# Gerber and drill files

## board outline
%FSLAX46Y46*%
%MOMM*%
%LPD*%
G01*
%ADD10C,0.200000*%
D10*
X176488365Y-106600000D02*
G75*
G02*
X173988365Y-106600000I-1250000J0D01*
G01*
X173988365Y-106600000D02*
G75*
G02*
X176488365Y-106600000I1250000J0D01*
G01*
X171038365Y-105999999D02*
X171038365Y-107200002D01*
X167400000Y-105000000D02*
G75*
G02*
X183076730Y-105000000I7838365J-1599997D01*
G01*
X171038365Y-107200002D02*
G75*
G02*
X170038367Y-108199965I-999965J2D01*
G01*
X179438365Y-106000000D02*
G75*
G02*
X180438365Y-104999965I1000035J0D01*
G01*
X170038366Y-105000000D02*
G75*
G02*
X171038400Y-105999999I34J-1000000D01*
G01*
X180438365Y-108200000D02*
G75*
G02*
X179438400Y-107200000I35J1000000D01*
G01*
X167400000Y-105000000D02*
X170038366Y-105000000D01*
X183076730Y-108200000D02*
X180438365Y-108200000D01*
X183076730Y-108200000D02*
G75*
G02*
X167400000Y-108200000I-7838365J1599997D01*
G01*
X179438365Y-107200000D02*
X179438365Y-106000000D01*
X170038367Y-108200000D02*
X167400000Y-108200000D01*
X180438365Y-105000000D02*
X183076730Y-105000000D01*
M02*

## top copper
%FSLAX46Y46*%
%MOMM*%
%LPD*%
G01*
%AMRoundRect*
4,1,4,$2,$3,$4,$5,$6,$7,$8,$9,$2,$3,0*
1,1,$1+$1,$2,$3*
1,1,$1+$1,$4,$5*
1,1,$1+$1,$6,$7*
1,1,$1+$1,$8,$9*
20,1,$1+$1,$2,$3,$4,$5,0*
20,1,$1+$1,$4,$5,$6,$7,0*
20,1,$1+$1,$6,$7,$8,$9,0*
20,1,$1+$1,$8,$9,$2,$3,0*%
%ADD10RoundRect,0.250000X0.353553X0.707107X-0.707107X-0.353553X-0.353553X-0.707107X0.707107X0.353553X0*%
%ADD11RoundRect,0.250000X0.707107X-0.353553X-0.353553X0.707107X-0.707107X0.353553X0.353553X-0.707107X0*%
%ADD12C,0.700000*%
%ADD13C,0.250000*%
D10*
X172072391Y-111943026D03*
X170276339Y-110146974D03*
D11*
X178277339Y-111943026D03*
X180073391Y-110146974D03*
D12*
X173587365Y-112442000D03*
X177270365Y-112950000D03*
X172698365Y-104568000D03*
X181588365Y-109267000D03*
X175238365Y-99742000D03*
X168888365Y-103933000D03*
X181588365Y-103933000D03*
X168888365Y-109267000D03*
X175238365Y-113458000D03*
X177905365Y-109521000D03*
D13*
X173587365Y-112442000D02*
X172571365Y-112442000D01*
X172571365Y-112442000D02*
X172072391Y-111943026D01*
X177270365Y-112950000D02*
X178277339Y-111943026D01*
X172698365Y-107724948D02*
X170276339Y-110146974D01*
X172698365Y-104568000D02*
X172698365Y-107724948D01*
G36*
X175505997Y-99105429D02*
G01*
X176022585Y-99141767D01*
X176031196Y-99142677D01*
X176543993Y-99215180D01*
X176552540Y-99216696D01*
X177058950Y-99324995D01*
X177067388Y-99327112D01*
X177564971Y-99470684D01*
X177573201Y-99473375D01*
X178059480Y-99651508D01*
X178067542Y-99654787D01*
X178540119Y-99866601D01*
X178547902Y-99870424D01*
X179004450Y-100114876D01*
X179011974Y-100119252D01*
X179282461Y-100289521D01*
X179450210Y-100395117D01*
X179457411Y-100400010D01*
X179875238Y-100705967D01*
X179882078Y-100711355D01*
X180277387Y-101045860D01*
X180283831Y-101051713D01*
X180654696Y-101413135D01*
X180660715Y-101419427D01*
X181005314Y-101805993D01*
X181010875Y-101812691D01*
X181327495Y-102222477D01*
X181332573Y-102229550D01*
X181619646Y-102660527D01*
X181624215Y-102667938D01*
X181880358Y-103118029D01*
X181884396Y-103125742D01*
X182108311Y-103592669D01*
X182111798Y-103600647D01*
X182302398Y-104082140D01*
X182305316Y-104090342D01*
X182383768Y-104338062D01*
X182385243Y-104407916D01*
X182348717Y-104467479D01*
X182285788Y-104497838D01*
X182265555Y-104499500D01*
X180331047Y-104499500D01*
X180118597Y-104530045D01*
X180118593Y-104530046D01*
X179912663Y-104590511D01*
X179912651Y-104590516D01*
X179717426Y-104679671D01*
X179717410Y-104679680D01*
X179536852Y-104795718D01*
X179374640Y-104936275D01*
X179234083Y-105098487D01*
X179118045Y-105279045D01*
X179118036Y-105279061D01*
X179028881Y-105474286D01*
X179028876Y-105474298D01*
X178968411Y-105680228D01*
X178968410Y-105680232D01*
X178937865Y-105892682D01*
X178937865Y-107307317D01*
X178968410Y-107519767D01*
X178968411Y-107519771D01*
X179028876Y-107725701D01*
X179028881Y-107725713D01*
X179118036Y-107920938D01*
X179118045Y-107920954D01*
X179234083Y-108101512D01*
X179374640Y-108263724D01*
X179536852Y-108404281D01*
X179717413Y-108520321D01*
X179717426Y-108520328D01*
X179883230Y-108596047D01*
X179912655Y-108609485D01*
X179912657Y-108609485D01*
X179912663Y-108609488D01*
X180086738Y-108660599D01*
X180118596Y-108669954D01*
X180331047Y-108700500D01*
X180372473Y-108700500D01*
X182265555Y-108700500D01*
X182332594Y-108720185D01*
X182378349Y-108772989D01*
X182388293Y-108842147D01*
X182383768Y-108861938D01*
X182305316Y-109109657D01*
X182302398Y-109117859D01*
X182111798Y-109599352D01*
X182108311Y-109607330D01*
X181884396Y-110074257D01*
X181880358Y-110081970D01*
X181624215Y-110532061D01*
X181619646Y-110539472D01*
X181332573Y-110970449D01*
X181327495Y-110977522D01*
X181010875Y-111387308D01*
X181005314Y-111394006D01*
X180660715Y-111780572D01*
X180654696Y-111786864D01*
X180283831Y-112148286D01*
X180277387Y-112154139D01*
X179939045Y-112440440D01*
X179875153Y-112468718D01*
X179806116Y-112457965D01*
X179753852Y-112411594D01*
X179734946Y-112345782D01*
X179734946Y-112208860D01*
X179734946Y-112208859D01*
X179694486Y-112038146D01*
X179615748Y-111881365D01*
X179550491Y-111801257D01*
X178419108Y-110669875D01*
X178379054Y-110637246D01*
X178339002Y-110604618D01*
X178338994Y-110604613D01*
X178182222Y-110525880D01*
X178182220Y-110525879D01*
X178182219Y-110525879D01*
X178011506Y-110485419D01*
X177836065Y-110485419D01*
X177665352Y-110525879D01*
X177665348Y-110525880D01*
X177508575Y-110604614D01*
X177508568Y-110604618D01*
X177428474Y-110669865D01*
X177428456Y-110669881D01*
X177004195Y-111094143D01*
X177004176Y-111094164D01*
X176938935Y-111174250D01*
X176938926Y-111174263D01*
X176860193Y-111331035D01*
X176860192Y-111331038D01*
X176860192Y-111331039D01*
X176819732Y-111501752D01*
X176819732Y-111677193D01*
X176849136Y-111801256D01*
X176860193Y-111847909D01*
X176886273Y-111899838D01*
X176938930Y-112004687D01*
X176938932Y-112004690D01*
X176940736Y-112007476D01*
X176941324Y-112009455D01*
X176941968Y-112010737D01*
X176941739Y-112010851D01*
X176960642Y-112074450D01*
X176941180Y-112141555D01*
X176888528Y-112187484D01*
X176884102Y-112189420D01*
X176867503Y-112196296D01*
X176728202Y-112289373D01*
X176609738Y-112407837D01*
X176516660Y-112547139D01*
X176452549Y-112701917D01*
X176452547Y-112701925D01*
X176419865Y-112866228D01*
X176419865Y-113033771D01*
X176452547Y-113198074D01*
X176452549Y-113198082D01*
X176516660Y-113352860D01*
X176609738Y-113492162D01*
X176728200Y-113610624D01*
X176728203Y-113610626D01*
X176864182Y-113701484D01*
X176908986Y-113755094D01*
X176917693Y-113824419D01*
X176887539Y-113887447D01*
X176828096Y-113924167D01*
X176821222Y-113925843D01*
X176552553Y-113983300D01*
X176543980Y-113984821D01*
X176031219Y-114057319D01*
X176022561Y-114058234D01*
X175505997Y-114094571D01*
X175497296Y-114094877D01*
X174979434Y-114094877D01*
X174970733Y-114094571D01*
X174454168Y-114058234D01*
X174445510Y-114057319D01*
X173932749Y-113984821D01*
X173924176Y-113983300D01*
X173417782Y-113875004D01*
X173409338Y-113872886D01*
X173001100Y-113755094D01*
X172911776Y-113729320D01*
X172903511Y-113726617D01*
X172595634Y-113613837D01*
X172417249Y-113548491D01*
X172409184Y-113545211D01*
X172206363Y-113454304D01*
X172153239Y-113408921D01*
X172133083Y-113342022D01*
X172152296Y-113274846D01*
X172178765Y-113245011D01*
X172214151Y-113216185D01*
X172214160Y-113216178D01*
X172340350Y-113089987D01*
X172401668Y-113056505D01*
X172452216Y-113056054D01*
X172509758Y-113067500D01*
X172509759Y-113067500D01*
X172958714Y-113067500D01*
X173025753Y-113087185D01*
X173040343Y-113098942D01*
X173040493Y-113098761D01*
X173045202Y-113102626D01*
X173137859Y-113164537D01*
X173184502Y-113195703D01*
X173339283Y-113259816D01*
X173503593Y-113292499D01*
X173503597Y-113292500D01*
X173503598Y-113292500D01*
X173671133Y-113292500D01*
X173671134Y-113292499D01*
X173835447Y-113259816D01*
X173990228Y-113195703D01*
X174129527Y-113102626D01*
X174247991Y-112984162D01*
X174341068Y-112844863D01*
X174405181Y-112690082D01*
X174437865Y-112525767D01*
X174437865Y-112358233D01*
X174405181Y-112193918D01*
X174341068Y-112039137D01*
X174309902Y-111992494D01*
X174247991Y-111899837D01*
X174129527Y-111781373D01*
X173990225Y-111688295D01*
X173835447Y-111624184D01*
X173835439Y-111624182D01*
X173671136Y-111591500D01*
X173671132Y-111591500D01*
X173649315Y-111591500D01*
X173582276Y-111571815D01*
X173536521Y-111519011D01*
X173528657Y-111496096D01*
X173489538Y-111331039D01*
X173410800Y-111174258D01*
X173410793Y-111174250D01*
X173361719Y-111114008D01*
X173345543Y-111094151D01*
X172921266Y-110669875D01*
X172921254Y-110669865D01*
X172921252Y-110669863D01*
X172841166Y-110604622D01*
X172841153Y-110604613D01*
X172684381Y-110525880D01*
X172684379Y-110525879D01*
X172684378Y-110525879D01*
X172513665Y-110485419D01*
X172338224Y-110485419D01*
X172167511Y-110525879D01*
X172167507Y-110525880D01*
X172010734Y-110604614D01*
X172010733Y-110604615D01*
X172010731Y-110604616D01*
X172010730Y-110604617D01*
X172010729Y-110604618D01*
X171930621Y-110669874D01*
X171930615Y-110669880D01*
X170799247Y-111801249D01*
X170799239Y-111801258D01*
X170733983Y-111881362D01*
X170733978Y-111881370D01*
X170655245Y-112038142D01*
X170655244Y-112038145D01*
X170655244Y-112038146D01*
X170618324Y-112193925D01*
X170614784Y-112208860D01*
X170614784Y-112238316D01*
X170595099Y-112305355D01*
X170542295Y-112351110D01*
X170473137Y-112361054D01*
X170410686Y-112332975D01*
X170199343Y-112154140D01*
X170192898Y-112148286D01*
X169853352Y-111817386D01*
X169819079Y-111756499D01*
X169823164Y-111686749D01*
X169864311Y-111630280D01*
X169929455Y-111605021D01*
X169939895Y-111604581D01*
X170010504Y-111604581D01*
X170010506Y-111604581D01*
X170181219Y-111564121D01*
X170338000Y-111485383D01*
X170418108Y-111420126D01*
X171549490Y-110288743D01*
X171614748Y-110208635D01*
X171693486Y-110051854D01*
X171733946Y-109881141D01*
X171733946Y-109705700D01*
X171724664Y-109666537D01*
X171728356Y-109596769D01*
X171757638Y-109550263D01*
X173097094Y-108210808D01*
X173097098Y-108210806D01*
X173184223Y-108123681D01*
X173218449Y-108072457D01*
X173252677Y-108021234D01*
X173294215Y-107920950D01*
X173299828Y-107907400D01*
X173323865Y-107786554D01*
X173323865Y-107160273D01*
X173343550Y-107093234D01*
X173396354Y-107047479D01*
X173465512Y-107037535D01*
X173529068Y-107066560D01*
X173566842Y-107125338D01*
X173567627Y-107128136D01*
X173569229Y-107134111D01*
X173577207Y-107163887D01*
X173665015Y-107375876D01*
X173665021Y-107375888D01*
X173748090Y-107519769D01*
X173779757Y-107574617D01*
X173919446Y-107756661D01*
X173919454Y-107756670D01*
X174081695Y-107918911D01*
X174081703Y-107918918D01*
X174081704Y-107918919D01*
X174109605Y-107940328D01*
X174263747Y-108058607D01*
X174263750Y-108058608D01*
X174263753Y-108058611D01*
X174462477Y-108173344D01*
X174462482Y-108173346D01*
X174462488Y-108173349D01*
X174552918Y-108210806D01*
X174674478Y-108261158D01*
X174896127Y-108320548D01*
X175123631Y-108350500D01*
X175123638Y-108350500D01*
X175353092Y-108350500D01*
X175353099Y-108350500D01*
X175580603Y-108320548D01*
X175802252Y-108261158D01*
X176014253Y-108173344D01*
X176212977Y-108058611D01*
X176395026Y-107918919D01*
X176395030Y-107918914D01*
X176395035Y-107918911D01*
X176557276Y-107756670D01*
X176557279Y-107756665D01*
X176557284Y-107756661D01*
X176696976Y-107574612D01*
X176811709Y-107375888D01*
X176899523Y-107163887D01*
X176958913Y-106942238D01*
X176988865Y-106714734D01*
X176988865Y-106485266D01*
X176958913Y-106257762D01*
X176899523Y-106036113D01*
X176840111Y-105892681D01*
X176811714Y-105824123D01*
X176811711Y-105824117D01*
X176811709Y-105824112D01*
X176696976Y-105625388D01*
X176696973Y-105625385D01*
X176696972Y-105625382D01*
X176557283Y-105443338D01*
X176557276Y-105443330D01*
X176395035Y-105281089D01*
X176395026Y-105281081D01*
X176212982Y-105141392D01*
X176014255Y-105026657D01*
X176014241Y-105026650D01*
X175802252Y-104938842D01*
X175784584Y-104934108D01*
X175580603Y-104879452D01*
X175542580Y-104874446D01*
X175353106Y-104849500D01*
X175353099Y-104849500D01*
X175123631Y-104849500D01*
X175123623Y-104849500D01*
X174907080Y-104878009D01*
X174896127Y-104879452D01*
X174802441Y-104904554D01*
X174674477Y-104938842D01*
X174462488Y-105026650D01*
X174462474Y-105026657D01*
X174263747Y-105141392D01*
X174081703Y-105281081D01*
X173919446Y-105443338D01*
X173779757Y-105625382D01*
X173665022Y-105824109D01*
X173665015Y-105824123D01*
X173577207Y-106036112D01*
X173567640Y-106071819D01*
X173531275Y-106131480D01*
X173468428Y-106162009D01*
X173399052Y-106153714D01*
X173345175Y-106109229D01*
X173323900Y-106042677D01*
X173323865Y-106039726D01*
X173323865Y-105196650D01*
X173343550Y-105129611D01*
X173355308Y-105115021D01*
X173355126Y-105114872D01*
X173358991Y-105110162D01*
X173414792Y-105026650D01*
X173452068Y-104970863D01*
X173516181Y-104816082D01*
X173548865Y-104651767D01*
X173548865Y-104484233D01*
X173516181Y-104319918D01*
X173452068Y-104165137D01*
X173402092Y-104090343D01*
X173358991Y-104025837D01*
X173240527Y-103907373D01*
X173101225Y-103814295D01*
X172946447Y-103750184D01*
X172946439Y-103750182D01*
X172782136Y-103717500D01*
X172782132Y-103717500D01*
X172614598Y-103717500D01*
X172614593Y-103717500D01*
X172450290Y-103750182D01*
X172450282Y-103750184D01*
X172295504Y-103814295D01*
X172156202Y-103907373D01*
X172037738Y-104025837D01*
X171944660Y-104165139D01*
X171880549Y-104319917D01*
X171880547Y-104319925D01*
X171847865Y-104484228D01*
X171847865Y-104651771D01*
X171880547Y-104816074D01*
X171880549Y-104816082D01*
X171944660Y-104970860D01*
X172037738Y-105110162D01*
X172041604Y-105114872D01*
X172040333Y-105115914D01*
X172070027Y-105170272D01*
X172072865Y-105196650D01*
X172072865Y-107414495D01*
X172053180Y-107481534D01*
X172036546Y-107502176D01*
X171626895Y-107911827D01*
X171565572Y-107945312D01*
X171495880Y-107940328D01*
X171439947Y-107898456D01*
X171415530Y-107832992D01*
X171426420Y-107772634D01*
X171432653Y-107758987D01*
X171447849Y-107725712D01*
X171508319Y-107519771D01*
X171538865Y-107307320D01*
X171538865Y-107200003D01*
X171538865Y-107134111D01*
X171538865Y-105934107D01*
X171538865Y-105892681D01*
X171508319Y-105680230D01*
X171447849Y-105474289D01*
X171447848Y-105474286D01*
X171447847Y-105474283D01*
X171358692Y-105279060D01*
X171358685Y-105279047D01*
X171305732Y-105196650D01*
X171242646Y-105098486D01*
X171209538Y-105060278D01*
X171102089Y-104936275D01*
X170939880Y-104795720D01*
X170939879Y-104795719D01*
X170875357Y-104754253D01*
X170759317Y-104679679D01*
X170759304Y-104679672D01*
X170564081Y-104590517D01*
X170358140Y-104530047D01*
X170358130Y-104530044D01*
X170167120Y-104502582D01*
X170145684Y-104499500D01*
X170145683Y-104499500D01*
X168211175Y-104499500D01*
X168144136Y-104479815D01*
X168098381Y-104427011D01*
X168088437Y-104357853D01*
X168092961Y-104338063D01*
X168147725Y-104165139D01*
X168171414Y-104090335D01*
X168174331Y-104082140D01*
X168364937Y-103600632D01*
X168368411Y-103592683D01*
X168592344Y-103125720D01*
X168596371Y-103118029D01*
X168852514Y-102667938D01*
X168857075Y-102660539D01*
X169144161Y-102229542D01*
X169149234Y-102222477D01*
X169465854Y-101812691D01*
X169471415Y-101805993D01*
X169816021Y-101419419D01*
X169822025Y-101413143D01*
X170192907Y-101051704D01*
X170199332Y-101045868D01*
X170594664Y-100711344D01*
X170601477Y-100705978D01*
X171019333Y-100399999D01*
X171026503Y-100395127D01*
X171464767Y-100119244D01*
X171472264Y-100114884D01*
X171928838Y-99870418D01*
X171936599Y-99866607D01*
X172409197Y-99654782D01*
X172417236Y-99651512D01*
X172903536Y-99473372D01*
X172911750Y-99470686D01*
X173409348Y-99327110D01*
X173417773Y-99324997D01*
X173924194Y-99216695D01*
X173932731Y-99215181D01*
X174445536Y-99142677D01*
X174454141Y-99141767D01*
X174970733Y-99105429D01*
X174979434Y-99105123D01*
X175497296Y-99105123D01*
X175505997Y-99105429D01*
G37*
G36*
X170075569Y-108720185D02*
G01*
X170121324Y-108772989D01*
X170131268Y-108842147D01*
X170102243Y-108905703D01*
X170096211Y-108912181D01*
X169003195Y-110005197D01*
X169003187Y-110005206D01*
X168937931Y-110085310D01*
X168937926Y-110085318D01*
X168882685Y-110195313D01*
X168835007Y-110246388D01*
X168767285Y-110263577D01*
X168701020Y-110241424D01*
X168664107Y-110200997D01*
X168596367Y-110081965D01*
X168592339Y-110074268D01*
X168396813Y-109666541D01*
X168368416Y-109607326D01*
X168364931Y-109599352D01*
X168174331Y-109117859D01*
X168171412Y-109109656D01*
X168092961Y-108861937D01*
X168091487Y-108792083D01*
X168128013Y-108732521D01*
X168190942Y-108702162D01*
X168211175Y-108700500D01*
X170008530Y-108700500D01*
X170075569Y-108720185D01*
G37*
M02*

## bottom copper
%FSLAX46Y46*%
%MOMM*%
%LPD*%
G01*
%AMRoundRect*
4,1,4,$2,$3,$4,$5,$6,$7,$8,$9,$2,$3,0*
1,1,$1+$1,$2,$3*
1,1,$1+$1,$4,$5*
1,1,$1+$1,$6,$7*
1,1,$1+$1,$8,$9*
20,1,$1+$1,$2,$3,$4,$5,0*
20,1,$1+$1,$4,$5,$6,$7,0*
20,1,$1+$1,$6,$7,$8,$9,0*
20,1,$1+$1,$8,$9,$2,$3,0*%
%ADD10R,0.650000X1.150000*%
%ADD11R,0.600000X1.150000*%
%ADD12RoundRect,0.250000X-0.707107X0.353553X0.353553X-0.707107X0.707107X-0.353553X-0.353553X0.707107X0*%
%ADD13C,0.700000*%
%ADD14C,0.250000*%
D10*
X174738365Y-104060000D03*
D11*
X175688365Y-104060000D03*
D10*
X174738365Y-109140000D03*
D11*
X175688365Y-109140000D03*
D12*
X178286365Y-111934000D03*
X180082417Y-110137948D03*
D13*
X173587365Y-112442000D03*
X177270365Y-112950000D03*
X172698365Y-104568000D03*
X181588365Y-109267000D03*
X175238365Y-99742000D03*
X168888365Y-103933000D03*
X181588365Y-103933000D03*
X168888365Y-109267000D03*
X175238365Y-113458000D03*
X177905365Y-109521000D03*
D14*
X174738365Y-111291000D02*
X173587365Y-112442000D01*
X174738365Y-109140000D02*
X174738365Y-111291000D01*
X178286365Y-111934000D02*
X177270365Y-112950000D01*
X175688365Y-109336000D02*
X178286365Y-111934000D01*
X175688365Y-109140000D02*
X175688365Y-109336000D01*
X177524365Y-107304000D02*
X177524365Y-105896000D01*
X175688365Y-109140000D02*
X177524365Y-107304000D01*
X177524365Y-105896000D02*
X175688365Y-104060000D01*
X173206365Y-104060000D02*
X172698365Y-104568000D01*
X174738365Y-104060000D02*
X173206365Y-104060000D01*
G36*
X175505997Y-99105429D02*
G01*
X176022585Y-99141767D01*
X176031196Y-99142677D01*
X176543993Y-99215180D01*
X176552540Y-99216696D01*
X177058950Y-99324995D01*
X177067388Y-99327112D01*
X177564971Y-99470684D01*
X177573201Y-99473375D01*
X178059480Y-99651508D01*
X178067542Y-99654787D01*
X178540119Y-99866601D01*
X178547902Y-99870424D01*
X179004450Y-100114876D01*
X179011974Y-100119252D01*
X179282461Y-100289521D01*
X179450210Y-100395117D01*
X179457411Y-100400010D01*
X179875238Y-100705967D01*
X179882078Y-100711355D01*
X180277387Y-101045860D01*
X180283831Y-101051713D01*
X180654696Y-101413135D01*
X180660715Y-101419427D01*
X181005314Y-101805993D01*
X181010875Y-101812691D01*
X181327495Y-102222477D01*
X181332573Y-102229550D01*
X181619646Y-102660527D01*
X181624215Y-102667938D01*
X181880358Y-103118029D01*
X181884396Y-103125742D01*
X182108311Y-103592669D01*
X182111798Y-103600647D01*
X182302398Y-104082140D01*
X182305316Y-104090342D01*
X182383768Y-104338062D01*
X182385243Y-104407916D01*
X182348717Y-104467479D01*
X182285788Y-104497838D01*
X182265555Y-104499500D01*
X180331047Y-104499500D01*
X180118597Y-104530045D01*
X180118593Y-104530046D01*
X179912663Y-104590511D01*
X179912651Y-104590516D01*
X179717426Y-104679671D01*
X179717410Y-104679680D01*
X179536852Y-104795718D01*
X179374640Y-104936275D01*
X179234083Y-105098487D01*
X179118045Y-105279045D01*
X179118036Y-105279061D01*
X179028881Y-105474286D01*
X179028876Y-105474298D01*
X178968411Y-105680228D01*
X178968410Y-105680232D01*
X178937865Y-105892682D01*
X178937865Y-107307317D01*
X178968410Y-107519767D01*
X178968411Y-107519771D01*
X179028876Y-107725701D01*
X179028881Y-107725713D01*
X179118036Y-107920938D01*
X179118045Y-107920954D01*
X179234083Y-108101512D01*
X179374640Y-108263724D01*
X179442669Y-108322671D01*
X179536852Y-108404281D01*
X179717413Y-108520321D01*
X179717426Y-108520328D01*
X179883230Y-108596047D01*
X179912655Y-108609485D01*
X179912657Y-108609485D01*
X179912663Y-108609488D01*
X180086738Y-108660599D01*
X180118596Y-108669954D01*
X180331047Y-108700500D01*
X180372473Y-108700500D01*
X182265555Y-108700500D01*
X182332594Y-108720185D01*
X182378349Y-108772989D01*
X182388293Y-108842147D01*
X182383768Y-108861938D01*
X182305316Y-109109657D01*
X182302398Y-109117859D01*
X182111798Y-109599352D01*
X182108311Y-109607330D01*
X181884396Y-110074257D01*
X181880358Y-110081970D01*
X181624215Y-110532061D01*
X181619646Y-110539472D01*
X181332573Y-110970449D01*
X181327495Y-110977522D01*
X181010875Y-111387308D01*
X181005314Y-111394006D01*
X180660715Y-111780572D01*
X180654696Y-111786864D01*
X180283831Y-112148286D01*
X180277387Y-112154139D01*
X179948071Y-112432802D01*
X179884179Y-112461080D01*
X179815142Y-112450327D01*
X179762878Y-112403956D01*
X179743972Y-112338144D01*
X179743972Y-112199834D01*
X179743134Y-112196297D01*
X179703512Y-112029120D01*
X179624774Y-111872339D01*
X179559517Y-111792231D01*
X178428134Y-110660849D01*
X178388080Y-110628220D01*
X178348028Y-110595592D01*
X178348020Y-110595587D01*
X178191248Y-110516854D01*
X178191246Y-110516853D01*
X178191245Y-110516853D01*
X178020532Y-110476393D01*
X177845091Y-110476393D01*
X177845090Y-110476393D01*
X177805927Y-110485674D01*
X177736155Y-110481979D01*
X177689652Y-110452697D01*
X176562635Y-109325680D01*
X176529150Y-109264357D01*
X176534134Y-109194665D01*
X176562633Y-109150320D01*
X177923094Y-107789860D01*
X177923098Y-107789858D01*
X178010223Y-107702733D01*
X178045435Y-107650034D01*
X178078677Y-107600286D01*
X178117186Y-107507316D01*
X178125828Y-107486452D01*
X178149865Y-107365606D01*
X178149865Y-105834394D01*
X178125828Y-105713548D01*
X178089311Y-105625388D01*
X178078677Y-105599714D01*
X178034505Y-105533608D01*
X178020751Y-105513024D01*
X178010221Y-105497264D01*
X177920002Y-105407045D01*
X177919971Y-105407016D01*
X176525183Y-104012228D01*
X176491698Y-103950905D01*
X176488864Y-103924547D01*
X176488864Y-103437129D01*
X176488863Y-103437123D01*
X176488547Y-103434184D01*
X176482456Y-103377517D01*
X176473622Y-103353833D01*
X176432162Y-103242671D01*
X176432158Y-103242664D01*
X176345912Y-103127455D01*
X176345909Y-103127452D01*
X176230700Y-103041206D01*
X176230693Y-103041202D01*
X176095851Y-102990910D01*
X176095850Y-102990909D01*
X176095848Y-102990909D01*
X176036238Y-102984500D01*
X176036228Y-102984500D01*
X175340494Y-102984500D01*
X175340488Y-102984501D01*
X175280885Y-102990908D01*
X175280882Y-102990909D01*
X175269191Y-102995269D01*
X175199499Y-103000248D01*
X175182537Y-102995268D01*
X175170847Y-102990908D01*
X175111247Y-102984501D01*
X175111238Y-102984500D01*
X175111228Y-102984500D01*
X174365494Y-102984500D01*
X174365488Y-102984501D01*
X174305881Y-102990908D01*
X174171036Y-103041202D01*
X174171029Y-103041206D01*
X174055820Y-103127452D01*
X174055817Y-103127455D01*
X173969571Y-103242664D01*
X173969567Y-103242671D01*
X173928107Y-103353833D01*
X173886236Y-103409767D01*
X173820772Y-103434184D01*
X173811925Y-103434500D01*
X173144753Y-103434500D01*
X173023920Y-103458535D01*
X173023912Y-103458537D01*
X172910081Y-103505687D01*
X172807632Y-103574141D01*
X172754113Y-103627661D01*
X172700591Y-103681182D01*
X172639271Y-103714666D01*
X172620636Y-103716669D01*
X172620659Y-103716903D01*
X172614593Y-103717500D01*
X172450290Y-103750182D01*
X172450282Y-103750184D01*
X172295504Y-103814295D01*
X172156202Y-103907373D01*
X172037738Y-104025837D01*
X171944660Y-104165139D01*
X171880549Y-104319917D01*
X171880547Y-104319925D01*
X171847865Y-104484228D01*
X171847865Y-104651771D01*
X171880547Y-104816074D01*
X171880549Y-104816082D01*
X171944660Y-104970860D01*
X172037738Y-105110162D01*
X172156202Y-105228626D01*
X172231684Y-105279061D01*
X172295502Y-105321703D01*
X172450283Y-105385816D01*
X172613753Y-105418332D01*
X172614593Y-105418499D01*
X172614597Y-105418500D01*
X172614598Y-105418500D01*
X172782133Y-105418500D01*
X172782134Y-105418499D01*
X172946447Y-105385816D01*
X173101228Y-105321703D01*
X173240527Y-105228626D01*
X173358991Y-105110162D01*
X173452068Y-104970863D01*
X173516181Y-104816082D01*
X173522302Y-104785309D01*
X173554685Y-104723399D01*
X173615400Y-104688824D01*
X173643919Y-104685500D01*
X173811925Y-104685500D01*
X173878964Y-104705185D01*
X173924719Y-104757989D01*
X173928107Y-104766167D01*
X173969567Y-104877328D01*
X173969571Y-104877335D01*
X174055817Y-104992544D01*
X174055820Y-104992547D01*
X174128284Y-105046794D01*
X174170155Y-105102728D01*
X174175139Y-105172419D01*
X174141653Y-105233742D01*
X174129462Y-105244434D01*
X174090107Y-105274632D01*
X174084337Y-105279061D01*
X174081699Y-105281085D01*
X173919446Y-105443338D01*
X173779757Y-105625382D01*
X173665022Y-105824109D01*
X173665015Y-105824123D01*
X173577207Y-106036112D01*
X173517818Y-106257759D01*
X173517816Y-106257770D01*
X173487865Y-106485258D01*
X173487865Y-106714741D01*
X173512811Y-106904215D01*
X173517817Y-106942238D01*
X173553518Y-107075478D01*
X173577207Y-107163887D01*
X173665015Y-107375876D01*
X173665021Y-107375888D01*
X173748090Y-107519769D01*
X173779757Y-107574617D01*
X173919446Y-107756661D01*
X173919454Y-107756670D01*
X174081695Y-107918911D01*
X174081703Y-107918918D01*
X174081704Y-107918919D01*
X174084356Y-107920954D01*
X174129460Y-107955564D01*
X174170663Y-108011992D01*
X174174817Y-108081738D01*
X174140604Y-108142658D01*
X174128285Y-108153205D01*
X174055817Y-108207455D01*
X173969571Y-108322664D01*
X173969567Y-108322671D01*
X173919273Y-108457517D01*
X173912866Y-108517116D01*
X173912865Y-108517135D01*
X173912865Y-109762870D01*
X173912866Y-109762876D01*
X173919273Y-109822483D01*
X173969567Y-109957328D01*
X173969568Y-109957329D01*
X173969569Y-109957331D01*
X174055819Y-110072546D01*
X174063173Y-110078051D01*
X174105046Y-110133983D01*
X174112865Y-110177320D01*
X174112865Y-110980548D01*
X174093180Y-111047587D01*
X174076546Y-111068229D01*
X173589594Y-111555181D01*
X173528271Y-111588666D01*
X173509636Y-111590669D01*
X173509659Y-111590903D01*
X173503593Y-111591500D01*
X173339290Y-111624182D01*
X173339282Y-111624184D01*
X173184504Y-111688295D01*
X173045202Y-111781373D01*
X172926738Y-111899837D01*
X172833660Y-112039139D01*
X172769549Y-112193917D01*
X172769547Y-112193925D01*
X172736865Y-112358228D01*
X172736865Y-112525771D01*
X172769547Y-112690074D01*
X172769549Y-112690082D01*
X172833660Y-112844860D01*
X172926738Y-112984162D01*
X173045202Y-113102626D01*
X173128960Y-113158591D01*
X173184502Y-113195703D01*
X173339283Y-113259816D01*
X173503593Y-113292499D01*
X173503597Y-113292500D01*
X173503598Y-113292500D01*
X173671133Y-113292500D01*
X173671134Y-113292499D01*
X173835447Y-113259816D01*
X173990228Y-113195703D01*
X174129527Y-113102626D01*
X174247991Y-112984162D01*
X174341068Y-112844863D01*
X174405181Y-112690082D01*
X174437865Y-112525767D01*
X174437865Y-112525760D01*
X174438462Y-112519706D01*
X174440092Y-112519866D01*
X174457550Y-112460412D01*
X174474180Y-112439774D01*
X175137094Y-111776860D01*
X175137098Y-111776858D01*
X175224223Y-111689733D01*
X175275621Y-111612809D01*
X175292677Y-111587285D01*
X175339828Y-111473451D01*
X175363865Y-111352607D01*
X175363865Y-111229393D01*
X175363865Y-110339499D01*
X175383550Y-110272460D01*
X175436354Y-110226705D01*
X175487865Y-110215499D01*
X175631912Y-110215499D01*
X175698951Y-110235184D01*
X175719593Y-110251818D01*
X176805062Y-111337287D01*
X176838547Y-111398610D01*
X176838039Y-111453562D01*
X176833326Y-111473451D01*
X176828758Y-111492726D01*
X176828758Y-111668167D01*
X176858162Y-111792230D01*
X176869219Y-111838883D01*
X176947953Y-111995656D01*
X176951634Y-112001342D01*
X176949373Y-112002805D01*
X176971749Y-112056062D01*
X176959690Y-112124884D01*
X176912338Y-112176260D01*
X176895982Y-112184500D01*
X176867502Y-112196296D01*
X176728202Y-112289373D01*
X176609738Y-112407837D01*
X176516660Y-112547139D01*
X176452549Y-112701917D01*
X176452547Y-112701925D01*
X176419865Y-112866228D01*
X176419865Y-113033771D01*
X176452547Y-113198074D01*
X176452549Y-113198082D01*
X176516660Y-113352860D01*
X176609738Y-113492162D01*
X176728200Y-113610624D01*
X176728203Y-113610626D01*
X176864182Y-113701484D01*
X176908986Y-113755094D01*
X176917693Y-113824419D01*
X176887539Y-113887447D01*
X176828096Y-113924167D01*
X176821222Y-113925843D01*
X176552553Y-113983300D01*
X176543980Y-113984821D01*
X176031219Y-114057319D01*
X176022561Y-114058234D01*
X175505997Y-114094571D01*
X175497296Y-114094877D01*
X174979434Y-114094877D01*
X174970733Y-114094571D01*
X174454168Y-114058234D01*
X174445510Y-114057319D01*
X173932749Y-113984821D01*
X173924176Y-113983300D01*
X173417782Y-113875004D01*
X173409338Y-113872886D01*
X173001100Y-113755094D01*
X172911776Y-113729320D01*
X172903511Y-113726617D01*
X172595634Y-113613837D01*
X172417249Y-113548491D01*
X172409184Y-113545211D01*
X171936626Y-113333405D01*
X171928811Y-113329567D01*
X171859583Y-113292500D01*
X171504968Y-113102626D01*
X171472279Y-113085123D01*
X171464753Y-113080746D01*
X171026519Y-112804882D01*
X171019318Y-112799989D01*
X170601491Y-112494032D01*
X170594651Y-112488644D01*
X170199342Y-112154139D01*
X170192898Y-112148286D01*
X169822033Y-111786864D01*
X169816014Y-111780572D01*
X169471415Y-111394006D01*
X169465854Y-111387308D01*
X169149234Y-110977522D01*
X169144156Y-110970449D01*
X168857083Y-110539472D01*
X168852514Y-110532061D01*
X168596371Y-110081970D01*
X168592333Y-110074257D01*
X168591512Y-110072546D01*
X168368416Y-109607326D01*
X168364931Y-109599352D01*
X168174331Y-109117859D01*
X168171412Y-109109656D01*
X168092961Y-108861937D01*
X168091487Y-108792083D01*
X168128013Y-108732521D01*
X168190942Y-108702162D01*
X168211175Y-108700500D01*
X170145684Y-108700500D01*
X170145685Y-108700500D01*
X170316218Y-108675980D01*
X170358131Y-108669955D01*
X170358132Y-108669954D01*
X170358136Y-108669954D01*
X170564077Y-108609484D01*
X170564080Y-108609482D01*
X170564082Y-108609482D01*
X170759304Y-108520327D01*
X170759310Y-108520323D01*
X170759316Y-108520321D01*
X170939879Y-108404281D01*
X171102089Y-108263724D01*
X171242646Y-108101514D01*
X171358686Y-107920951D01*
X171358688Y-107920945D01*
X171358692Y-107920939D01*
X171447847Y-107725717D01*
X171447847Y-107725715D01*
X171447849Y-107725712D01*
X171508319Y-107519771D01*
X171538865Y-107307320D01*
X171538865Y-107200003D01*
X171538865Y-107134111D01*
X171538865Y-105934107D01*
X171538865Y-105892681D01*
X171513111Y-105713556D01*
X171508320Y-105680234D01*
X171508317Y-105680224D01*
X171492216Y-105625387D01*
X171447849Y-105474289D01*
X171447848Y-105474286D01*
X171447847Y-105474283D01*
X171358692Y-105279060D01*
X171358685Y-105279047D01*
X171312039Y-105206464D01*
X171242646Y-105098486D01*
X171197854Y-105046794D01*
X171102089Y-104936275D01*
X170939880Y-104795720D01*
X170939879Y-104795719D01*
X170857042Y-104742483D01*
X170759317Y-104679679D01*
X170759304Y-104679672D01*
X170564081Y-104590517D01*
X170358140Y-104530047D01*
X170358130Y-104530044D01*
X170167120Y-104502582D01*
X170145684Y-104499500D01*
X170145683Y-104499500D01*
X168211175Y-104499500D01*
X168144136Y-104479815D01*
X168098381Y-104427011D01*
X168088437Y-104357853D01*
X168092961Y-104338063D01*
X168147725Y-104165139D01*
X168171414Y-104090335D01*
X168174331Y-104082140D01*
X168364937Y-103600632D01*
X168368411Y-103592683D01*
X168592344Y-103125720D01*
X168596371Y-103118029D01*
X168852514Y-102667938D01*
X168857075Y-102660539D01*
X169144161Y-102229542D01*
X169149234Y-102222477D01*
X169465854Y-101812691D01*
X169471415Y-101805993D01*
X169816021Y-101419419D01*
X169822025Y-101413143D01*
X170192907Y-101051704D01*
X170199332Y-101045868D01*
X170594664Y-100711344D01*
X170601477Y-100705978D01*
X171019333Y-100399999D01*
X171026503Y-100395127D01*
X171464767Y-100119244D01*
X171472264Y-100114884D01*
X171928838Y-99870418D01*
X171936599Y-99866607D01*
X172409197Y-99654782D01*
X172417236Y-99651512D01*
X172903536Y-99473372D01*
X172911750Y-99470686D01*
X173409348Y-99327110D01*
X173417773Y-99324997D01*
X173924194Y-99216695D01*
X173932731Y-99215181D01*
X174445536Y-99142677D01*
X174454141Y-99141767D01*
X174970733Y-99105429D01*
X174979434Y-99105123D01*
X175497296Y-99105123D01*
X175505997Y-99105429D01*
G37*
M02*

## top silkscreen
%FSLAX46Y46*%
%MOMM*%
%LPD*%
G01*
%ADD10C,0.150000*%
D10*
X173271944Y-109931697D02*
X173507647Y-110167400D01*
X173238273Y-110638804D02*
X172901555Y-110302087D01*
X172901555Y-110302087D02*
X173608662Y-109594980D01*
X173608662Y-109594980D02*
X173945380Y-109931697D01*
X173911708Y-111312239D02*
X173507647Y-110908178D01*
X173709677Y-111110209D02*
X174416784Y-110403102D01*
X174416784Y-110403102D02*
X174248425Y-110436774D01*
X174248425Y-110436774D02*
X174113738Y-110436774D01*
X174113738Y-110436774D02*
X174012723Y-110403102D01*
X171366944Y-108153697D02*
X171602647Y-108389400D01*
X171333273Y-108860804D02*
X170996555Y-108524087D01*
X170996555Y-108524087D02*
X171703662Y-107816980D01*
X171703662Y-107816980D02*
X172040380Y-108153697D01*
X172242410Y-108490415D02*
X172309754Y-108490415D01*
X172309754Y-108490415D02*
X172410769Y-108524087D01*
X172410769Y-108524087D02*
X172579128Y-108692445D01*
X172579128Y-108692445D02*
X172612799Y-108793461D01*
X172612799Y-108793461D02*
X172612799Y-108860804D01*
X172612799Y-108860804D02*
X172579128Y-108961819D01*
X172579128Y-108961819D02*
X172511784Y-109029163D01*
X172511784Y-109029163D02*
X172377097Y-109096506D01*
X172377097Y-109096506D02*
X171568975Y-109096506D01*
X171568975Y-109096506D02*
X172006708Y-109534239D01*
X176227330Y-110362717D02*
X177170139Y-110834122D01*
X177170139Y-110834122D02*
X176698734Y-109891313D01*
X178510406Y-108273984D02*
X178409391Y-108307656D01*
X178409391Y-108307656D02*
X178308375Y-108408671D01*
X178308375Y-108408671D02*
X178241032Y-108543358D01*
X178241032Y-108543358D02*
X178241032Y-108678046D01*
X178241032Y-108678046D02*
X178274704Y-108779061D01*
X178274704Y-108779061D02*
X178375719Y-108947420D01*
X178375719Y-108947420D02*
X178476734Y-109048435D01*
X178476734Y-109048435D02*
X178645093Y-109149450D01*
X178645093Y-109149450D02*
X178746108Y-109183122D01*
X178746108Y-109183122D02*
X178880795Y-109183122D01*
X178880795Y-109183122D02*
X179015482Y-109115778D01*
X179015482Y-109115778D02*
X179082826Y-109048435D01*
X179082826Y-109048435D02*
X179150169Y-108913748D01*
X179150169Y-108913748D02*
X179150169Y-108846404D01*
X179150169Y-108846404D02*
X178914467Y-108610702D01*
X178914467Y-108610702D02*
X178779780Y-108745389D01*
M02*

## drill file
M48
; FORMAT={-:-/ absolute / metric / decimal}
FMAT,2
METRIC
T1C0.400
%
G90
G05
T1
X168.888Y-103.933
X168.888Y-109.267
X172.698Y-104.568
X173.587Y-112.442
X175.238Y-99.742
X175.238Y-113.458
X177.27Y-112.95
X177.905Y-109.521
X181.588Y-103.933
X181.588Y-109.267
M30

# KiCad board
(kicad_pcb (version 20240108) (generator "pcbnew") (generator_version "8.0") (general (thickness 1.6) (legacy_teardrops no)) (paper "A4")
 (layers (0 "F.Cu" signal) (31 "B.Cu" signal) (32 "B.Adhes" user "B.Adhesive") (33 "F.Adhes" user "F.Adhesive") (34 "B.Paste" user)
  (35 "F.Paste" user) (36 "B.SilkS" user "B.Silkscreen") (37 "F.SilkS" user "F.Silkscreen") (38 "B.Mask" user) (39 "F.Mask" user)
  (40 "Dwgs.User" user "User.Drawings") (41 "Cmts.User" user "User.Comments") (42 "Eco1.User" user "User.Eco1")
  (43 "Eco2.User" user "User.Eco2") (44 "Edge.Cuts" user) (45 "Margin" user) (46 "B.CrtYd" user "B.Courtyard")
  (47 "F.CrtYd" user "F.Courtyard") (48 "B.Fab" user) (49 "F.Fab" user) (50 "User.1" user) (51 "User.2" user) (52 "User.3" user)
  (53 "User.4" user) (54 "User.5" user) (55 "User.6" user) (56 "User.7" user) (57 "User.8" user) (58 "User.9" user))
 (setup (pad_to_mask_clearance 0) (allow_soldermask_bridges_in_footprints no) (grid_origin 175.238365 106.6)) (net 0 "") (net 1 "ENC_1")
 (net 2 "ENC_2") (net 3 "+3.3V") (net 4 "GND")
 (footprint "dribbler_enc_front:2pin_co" (layer "F.Cu") (at 171.174365 111.045 135)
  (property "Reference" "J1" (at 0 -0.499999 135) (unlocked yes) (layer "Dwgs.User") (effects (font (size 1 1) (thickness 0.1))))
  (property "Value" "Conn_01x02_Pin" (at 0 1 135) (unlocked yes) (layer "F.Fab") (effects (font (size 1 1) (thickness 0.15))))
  (pad "1" smd roundrect (at -1.270001 0 225) (size 2 1) (layers "F.Cu" "F.Paste" "F.Mask") (roundrect_rratio 0.25) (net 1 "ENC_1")
   (thermal_bridge_angle 45))
  (pad "2" smd roundrect (at 1.270001 0 225) (size 2 1) (layers "F.Cu" "F.Paste" "F.Mask") (roundrect_rratio 0.25) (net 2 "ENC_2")
   (thermal_bridge_angle 45)))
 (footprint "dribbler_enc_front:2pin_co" (layer "F.Cu") (at 179.175365 111.045 45)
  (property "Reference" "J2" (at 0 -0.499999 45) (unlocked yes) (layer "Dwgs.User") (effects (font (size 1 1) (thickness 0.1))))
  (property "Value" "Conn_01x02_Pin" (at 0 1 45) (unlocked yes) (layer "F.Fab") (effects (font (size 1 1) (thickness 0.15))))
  (pad "1" smd roundrect (at -1.270001 0 135) (size 2 1) (layers "F.Cu" "F.Paste" "F.Mask") (roundrect_rratio 0.25) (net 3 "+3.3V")
   (thermal_bridge_angle 45))
  (pad "2" smd roundrect (at 1.270001 0 135) (size 2 1) (layers "F.Cu" "F.Paste" "F.Mask") (roundrect_rratio 0.25) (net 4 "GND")
   (thermal_bridge_angle 45)))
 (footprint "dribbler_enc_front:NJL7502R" (layer "B.Cu") (at 175.238365 104.06 90)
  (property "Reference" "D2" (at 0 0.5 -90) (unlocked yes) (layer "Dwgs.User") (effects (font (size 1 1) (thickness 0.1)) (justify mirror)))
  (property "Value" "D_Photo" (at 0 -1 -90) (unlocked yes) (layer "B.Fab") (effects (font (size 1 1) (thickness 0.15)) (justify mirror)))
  (pad "1" smd rect (at 0 -0.5 90) (size 1.15 0.65) (layers "B.Cu" "B.Paste" "B.Mask") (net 2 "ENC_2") (thermal_bridge_angle 45))
  (pad "2" smd rect (at 0 0.45 90) (size 1.15 0.6) (layers "B.Cu" "B.Paste" "B.Mask") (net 3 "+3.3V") (thermal_bridge_angle 45)))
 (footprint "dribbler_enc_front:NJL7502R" (layer "B.Cu") (at 175.238365 109.14 90)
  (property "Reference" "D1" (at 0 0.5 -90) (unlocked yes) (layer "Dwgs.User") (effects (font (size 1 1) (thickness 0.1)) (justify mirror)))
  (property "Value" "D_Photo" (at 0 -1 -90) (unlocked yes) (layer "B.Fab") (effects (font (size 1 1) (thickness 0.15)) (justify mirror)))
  (pad "1" smd rect (at 0 -0.5 90) (size 1.15 0.65) (layers "B.Cu" "B.Paste" "B.Mask") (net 1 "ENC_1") (thermal_bridge_angle 45))
  (pad "2" smd rect (at 0 0.45 90) (size 1.15 0.6) (layers "B.Cu" "B.Paste" "B.Mask") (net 3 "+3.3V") (thermal_bridge_angle 45)))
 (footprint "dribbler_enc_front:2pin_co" (layer "B.Cu") (at 179.184391 111.035974 45)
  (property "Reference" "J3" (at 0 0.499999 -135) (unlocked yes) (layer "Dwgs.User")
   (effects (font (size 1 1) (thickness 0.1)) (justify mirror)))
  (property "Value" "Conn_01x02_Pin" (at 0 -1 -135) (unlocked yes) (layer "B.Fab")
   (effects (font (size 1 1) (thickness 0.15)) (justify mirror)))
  (pad "1" smd roundrect (at -1.270001 0 315) (size 2 1) (layers "B.Cu" "B.Paste" "B.Mask") (roundrect_rratio 0.25) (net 3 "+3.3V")
   (thermal_bridge_angle 45))
  (pad "2" smd roundrect (at 1.270001 0 315) (size 2 1) (layers "B.Cu" "B.Paste" "B.Mask") (roundrect_rratio 0.25) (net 4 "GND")
   (thermal_bridge_angle 45)))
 (gr_circle (center 175.238365 106.6) (end 176.488365 106.6) (stroke (width 0.2) (type default)) (fill none) (layer "Edge.Cuts"))
 (gr_line (start 171.038365 105.999999) (end 171.038365 107.200002) (stroke (width 0.2) (type default)) (layer "Edge.Cuts"))
 (gr_arc (start 167.4 105) (mid 175.238365 98.6) (end 183.07673 105) (stroke (width 0.2) (type default)) (layer "Edge.Cuts"))
 (gr_arc (start 171.038365 107.200002) (mid 170.745472 107.907107) (end 170.038367 108.2) (stroke (width 0.2) (type default))
  (layer "Edge.Cuts"))
 (gr_arc (start 179.438365 106) (mid 179.731258 105.292893) (end 180.438365 105) (stroke (width 0.2) (type default)) (layer "Edge.Cuts"))
 (gr_arc (start 170.038366 105) (mid 170.745472 105.292893) (end 171.038365 105.999999) (stroke (width 0.2) (type default))
  (layer "Edge.Cuts"))
 (gr_arc (start 180.438365 108.2) (mid 179.731258 107.907107) (end 179.438365 107.2) (stroke (width 0.2) (type default)) (layer "Edge.Cuts"))
 (gr_line (start 167.4 105) (end 170.038366 105) (stroke (width 0.2) (type default)) (layer "Edge.Cuts"))
 (gr_line (start 183.07673 108.2) (end 180.438365 108.2) (stroke (width 0.2) (type default)) (layer "Edge.Cuts"))
 (gr_arc (start 183.07673 108.2) (mid 175.238365 114.6) (end 167.4 108.2) (stroke (width 0.2) (type default)) (layer "Edge.Cuts"))
 (gr_line (start 179.438365 107.2) (end 179.438365 106) (stroke (width 0.2) (type default)) (layer "Edge.Cuts"))
 (gr_line (start 170.038367 108.2) (end 167.4 108.2) (stroke (width 0.2) (type default)) (layer "Edge.Cuts"))
 (gr_line (start 180.438365 105) (end 183.07673 105) (stroke (width 0.2) (type default)) (layer "Edge.Cuts"))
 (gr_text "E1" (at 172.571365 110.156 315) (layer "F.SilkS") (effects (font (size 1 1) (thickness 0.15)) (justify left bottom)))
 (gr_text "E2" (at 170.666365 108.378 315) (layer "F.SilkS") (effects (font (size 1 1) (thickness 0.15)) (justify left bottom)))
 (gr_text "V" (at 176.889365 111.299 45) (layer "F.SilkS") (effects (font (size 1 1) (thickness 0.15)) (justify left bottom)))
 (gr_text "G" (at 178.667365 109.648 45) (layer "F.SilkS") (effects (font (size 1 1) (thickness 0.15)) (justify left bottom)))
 (segment (start 173.587365 112.442) (end 172.571365 112.442) (width 0.25) (layer "F.Cu") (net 1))
 (segment (start 172.571365 112.442) (end 172.072391 111.943026) (width 0.25) (layer "F.Cu") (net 1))
 (via (at 173.587365 112.442) (size 0.7) (drill 0.4) (layers "F.Cu" "B.Cu") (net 1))
 (segment (start 174.738365 111.291) (end 173.587365 112.442) (width 0.25) (layer "B.Cu") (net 1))
 (segment (start 174.738365 109.14) (end 174.738365 111.291) (width 0.25) (layer "B.Cu") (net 1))
 (segment (start 177.270365 112.95) (end 178.277339 111.943026) (width 0.25) (layer "F.Cu") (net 3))
 (via (at 177.270365 112.95) (size 0.7) (drill 0.4) (layers "F.Cu" "B.Cu") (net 3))
 (segment (start 178.286365 111.934) (end 177.270365 112.95) (width 0.25) (layer "B.Cu") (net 3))
 (segment (start 175.688365 109.336) (end 178.286365 111.934) (width 0.25) (layer "B.Cu") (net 3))
 (segment (start 175.688365 109.14) (end 175.688365 109.336) (width 0.25) (layer "B.Cu") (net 3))
 (segment (start 177.524365 107.304) (end 177.524365 105.896) (width 0.25) (layer "B.Cu") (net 3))
 (segment (start 175.688365 109.14) (end 177.524365 107.304) (width 0.25) (layer "B.Cu") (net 3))
 (segment (start 177.524365 105.896) (end 175.688365 104.06) (width 0.25) (layer "B.Cu") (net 3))
 (segment (start 172.698365 107.724948) (end 170.276339 110.146974) (width 0.25) (layer "F.Cu") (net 2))
 (segment (start 172.698365 104.568) (end 172.698365 107.724948) (width 0.25) (layer "F.Cu") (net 2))
 (via (at 172.698365 104.568) (size 0.7) (drill 0.4) (layers "F.Cu" "B.Cu") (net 2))
 (segment (start 173.206365 104.06) (end 172.698365 104.568) (width 0.25) (layer "B.Cu") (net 2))
 (segment (start 174.738365 104.06) (end 173.206365 104.06) (width 0.25) (layer "B.Cu") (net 2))
 (via (at 181.588365 109.267) (size 0.7) (drill 0.4) (layers "F.Cu" "B.Cu") (free yes) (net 4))
 (via (at 175.238365 99.742) (size 0.7) (drill 0.4) (layers "F.Cu" "B.Cu") (free yes) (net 4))
 (via (at 168.888365 103.933) (size 0.7) (drill 0.4) (layers "F.Cu" "B.Cu") (free yes) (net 4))
 (via (at 181.588365 103.933) (size 0.7) (drill 0.4) (layers "F.Cu" "B.Cu") (free yes) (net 4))
 (via (at 168.888365 109.267) (size 0.7) (drill 0.4) (layers "F.Cu" "B.Cu") (free yes) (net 4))
 (via (at 175.238365 113.458) (size 0.7) (drill 0.4) (layers "F.Cu" "B.Cu") (free yes) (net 4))
 (via (at 177.905365 109.521) (size 0.7) (drill 0.4) (layers "F.Cu" "B.Cu") (free yes) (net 4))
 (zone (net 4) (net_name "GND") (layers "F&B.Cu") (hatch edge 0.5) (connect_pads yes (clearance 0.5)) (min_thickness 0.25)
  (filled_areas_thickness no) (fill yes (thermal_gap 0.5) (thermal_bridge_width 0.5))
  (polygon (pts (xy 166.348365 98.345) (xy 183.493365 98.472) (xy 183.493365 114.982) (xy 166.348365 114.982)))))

